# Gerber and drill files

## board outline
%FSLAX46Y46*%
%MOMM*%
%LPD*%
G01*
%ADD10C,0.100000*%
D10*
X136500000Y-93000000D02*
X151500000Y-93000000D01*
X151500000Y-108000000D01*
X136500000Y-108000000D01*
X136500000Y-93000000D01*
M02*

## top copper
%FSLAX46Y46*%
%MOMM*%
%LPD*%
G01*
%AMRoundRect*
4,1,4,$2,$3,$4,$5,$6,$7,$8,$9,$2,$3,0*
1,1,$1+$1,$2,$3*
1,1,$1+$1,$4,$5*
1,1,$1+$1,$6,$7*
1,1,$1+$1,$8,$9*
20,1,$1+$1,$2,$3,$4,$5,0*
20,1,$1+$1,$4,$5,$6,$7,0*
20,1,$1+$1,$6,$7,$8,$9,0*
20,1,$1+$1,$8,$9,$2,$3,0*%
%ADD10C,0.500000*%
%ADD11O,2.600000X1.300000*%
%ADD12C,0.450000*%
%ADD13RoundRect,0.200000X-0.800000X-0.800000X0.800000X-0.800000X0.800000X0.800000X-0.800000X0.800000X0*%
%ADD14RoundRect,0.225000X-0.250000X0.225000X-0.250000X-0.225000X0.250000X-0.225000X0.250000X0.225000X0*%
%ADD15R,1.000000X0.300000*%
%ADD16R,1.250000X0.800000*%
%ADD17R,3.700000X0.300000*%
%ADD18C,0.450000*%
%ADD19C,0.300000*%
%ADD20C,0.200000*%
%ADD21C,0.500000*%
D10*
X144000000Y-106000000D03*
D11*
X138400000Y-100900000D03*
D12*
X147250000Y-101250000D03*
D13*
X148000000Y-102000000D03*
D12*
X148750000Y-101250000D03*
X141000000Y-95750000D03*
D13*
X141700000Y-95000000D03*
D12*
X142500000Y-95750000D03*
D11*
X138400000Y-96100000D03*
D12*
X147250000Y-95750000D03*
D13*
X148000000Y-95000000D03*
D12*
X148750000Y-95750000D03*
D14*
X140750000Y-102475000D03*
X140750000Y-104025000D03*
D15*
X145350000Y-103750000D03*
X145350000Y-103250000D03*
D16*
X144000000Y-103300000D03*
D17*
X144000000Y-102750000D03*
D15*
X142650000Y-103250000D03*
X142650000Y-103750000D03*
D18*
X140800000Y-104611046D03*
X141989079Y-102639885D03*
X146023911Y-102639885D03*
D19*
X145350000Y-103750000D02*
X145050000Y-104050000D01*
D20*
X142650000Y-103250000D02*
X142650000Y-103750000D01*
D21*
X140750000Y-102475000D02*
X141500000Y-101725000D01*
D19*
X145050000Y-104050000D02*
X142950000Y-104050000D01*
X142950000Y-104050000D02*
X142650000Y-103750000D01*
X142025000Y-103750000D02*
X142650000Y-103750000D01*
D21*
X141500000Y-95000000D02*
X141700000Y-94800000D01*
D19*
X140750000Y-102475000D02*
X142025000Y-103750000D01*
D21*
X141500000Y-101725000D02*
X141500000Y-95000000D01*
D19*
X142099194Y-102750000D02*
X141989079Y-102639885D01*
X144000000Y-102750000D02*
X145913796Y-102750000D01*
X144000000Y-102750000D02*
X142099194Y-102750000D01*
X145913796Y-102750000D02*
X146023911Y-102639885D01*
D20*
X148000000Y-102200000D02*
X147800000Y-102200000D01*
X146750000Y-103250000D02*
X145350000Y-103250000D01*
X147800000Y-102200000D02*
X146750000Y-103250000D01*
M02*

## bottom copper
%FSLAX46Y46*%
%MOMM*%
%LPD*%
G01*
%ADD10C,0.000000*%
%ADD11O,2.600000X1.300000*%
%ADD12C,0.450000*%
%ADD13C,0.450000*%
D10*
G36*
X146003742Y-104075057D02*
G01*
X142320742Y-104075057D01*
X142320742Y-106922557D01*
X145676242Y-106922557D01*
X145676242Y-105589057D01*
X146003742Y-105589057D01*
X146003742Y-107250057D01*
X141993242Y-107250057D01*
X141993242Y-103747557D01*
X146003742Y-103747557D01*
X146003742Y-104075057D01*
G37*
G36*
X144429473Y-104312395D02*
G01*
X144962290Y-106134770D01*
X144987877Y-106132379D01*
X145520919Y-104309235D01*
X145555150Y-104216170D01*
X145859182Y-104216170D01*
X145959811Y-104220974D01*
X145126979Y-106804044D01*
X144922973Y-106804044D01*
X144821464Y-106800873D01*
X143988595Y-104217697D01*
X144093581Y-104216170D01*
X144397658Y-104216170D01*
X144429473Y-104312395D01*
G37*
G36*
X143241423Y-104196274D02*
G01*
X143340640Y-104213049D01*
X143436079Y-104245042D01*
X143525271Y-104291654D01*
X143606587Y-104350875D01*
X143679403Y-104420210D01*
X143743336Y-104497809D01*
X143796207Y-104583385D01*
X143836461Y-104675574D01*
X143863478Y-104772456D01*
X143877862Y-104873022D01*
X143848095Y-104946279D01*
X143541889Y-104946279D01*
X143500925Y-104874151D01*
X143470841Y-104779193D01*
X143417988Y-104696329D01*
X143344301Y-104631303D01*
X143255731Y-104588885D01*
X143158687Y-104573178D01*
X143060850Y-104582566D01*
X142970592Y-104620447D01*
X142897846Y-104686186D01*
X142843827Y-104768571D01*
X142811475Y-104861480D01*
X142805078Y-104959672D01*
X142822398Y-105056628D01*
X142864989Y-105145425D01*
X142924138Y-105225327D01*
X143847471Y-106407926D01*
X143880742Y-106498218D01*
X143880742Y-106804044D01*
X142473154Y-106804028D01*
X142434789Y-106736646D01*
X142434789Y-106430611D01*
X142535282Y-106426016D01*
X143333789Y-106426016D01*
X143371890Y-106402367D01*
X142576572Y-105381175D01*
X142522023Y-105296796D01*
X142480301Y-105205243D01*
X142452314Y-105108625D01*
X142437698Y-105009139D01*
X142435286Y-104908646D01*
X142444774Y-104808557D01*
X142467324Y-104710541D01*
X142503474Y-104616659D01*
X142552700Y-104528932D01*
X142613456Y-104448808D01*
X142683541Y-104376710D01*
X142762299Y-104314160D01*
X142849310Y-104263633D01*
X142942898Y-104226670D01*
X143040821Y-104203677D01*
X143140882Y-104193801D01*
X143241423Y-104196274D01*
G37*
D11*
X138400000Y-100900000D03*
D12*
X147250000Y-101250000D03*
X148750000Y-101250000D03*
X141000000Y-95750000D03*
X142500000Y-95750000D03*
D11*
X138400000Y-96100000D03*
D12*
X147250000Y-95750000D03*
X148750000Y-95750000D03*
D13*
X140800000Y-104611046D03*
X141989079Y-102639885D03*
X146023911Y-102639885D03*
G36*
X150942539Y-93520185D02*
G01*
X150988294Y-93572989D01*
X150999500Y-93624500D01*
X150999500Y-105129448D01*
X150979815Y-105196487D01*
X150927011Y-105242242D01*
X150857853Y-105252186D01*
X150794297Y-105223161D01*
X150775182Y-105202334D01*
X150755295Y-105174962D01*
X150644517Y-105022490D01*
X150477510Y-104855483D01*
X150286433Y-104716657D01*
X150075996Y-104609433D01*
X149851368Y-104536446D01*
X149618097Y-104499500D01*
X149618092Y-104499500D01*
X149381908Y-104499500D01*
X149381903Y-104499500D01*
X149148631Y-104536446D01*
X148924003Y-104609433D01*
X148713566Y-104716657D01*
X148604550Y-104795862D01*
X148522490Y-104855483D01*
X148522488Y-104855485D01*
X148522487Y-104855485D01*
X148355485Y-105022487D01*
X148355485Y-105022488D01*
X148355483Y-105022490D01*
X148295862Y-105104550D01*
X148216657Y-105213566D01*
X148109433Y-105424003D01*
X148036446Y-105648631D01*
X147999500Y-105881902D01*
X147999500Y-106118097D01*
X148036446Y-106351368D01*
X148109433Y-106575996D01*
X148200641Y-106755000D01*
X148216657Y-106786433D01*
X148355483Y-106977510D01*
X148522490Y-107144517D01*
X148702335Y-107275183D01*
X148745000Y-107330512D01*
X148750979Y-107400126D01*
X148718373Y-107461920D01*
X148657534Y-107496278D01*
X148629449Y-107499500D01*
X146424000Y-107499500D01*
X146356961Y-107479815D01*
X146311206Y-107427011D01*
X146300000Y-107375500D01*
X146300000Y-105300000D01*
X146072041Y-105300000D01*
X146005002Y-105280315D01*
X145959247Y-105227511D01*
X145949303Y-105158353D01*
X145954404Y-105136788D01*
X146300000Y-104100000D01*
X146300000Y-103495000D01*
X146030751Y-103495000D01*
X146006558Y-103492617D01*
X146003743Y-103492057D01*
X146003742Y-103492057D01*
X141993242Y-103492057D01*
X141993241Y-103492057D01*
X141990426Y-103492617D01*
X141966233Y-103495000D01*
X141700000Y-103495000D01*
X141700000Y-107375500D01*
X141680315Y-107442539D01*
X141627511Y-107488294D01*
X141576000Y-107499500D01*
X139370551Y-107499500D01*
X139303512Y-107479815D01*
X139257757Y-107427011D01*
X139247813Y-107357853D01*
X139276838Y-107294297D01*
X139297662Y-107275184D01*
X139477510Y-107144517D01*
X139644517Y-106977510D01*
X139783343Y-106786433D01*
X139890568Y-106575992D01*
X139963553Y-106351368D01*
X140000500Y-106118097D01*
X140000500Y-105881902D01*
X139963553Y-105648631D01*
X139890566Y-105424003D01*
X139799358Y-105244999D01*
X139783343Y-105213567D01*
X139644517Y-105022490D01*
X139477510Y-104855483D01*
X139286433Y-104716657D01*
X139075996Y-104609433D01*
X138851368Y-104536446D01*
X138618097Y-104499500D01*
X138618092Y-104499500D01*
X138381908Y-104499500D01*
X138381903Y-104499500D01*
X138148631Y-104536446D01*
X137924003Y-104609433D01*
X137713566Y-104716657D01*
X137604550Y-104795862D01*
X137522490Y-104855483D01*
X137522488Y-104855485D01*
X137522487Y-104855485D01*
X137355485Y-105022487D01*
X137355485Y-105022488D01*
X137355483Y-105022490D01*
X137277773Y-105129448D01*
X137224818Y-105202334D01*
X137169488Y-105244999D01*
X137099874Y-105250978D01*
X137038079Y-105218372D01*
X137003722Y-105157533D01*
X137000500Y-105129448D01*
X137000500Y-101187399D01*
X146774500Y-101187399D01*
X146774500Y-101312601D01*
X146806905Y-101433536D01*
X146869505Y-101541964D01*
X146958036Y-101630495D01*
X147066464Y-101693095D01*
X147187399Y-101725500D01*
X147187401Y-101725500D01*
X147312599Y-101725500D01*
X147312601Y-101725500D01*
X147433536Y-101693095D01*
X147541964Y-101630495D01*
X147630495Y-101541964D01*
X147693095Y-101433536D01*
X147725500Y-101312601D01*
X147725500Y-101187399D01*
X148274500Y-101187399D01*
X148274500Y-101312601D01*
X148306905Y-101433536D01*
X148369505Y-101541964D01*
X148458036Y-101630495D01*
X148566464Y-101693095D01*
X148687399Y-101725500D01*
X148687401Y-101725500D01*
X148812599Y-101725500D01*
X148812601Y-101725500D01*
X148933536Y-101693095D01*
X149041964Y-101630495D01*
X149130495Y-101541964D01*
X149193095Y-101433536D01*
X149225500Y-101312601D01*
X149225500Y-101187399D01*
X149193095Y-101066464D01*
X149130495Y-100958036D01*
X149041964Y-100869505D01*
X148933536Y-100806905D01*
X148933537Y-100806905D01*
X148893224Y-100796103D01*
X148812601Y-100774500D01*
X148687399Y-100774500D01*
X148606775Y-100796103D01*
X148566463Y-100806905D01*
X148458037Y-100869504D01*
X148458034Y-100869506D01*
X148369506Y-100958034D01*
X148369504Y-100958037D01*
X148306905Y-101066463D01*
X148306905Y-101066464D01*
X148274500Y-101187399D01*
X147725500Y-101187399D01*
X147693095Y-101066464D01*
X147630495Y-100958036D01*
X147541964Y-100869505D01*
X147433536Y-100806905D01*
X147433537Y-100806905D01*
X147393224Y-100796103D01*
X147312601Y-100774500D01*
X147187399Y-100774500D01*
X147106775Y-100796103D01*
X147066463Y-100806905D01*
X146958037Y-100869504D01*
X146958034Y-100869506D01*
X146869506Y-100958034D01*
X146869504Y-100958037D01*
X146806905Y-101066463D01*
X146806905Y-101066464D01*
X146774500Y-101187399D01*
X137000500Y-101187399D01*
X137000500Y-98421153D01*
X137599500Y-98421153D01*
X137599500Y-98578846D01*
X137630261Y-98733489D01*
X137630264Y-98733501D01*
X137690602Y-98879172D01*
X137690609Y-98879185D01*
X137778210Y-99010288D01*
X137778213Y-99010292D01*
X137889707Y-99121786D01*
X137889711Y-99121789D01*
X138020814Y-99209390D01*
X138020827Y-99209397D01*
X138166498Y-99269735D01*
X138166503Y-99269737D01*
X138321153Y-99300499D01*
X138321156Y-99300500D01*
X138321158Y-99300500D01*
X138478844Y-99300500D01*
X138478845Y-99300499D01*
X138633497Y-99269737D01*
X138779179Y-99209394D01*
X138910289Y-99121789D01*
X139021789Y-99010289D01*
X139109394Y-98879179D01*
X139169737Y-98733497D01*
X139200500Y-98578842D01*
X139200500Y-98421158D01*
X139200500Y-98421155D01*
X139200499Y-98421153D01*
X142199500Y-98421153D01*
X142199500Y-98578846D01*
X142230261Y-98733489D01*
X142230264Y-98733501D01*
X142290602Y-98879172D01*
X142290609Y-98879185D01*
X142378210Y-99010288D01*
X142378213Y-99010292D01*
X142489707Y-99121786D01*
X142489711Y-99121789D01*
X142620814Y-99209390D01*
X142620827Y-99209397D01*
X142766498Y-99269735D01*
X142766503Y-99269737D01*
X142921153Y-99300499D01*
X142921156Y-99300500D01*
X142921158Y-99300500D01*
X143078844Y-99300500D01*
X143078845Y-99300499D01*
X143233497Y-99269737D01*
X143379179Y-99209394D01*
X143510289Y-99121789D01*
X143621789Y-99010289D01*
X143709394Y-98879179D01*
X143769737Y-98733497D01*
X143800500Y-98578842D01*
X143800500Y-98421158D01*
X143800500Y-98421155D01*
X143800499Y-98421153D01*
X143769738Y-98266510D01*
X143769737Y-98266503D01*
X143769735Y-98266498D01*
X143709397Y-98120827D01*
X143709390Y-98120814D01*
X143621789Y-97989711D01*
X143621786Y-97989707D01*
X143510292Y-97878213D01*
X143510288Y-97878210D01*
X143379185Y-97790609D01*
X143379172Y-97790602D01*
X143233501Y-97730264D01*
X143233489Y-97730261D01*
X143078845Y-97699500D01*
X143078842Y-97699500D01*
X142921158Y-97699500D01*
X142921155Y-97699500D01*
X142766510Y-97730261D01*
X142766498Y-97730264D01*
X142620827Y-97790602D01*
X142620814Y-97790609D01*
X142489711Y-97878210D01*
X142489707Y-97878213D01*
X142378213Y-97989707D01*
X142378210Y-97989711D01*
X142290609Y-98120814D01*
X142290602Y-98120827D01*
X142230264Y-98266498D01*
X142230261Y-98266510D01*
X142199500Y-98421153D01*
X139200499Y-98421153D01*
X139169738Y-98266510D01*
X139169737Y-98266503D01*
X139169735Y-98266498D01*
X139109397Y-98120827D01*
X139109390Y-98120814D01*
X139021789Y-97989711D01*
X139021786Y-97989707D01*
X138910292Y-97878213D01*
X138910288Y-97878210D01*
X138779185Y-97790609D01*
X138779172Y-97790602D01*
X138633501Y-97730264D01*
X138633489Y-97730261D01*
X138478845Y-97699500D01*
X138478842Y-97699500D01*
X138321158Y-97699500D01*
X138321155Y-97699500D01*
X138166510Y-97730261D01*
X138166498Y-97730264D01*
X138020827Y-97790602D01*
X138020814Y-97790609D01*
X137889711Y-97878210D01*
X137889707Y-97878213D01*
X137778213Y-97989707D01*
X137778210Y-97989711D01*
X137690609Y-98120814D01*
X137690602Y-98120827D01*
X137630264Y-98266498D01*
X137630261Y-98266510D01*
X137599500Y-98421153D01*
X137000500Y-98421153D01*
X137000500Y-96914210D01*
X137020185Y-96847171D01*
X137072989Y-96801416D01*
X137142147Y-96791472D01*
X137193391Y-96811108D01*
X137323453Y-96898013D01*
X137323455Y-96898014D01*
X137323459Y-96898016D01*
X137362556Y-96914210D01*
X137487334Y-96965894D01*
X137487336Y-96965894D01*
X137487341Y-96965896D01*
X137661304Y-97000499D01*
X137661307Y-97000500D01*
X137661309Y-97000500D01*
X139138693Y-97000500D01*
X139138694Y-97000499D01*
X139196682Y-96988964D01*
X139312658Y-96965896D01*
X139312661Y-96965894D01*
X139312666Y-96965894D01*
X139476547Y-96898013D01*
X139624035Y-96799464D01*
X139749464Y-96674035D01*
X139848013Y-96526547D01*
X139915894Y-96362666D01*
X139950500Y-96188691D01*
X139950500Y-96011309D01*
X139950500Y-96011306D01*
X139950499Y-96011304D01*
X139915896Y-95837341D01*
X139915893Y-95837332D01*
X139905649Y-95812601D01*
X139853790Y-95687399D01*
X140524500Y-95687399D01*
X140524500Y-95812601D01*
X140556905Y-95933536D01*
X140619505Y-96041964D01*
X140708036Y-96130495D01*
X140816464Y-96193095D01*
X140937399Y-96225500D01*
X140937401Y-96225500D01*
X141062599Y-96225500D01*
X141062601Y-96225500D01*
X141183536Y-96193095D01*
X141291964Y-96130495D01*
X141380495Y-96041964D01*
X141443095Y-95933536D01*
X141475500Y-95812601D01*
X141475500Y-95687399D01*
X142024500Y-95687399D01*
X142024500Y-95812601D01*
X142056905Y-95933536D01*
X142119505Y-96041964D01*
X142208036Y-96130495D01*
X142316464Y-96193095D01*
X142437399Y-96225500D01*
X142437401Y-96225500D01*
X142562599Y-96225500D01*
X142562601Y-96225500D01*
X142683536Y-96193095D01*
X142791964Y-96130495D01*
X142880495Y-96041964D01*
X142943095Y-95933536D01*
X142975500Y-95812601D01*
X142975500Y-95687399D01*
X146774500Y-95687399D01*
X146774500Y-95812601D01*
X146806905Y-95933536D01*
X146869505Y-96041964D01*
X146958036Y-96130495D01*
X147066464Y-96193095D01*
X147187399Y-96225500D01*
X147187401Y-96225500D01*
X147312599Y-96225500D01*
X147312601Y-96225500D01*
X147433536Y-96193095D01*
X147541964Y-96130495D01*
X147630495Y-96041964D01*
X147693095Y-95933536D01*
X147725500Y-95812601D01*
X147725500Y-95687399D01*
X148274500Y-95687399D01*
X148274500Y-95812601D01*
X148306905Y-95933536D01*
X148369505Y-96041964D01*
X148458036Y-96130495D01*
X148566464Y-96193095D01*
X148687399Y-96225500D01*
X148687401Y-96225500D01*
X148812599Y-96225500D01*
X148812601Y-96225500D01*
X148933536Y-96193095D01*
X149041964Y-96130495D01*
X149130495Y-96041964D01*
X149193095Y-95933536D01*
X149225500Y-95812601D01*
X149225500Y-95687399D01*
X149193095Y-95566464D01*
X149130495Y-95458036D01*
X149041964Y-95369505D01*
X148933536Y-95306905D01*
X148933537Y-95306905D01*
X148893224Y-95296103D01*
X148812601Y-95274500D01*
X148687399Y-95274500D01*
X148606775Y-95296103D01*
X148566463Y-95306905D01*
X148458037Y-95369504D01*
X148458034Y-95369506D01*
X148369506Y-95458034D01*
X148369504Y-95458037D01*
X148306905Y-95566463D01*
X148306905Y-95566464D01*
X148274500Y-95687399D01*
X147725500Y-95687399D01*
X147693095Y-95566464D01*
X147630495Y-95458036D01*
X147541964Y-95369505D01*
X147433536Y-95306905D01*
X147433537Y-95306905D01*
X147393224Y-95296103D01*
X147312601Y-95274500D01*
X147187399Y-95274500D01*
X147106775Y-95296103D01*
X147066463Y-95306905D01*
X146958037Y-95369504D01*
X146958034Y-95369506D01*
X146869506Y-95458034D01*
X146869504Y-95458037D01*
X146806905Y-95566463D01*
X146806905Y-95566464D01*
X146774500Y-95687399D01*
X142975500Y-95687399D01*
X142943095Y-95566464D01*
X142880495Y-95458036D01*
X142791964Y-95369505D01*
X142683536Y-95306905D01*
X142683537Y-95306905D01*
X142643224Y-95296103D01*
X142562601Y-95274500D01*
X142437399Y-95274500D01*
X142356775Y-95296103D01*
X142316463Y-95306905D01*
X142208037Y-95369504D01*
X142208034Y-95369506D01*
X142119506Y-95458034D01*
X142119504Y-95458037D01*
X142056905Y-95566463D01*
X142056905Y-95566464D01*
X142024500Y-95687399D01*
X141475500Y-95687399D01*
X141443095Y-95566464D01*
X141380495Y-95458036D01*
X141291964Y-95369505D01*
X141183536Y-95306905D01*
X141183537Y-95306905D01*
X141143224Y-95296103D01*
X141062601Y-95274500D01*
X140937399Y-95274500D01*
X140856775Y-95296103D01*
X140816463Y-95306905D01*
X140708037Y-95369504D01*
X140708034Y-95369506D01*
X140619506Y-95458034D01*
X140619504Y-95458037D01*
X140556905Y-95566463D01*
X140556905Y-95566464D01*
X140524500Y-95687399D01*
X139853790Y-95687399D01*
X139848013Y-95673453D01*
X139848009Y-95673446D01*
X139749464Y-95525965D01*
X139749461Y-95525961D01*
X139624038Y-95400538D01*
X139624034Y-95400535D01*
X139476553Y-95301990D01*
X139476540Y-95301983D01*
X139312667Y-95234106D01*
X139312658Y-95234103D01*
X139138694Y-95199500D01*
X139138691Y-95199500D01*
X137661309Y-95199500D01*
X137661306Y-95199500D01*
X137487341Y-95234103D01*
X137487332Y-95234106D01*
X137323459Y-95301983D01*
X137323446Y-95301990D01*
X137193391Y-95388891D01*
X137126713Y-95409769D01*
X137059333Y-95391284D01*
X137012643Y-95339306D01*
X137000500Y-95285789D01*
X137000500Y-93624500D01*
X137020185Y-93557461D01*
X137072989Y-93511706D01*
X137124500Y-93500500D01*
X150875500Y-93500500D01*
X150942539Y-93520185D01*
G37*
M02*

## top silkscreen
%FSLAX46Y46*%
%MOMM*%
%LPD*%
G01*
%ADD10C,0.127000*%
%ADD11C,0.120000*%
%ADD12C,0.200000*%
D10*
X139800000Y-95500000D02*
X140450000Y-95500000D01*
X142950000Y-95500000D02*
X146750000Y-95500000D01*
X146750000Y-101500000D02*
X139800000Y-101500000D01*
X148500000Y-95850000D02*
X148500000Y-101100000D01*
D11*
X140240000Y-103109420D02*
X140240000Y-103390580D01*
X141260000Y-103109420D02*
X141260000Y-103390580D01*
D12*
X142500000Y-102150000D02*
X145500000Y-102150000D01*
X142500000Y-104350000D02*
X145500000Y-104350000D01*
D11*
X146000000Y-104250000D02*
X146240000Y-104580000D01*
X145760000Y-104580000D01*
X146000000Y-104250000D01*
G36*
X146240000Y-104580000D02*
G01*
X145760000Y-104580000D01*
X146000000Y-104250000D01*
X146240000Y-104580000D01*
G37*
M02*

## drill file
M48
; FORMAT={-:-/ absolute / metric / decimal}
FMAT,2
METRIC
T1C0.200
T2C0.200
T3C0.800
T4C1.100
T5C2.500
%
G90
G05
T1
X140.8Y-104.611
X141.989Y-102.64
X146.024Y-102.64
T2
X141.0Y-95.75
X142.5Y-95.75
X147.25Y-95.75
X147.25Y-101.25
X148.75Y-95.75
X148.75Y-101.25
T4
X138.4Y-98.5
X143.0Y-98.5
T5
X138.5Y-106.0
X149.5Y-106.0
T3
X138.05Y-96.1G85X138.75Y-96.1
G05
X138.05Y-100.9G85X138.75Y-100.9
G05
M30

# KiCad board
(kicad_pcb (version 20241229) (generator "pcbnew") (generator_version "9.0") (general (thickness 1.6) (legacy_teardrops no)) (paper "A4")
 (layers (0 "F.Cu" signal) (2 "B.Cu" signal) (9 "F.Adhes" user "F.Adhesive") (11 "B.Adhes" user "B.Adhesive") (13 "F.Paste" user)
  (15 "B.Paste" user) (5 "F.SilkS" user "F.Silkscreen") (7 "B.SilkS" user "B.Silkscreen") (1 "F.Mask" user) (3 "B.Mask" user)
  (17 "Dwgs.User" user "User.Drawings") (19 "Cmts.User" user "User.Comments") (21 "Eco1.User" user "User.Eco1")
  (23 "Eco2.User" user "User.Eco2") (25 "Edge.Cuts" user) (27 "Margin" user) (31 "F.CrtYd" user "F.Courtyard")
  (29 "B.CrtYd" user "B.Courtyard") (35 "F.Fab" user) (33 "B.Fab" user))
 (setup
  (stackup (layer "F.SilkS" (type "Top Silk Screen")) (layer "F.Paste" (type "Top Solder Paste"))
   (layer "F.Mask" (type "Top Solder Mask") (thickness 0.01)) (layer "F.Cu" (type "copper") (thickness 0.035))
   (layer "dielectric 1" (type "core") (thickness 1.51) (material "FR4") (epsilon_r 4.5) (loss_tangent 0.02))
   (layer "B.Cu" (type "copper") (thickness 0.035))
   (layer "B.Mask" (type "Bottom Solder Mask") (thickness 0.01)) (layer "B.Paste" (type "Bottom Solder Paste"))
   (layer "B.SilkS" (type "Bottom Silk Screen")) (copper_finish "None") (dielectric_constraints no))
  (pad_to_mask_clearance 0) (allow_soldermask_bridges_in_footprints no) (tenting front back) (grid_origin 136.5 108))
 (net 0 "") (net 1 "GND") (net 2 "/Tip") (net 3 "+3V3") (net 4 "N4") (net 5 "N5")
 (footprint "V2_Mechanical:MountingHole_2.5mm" (layer "F.Cu") (at 138.5 106)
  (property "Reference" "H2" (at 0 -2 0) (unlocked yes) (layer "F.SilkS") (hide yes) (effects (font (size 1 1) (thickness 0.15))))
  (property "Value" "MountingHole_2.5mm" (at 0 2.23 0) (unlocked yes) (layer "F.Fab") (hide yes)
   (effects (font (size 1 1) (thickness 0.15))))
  (pad "" np_thru_hole circle (at 0 0) (size 2.5 2.5) (drill 2.5) (layers "*.Mask")))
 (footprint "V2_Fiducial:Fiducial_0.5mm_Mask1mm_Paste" (layer "F.Cu") (at 144 106)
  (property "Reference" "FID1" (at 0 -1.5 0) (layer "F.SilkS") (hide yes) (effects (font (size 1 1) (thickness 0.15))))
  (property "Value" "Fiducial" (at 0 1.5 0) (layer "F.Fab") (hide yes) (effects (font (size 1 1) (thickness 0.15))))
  (pad "" smd circle (at 0 0) (size 0.5 0.5) (layers "F.Cu" "F.Mask" "F.Paste") (solder_mask_margin 0.25) (clearance 0.25)))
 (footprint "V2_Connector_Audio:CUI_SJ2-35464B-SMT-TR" (layer "F.Cu") (at 142.5 98.5)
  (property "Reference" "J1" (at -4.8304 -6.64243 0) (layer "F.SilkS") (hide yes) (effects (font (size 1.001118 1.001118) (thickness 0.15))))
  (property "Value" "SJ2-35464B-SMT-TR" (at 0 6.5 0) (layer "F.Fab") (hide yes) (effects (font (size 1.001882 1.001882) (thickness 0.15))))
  (fp_line (start -2.7 -3) (end -2.05 -3) (stroke (width 0.127) (type solid)) (layer "F.SilkS"))
  (fp_line (start 0.45 -3) (end 4.25 -3) (stroke (width 0.127) (type solid)) (layer "F.SilkS"))
  (fp_line (start 4.25 3) (end -2.7 3) (stroke (width 0.127) (type solid)) (layer "F.SilkS"))
  (fp_line (start 6 -2.65) (end 6 2.6) (stroke (width 0.127) (type solid)) (layer "F.SilkS"))
  (pad "" np_thru_hole circle (at -4.1 0) (size 1.1 1.1) (drill 1.1) (layers "*.Cu" "*.Mask"))
  (pad "" smd roundrect (at -0.8 -3.7) (size 2 1.6) (layers "F.Mask") (roundrect_rratio 0.1) (solder_mask_margin 0.102))
  (pad "" smd roundrect (at -0.75 -3.825) (size 2.5 1.85) (layers "F.Paste") (roundrect_rratio 0.25) (solder_mask_margin 0.102))
  (pad "" np_thru_hole circle (at 0.5 0) (size 1.1 1.1) (drill 1.1) (layers "*.Cu" "*.Mask"))
  (pad "" smd roundrect (at 5.5 -3.825) (size 2.5 1.85) (layers "F.Paste") (roundrect_rratio 0.25) (solder_mask_margin 0.102))
  (pad "" smd roundrect (at 5.5 -3.7) (size 2 1.6) (layers "F.Mask") (roundrect_rratio 0.1) (solder_mask_margin 0.102))
  (pad "" smd roundrect (at 5.5 3.7) (size 2 1.6) (layers "F.Mask") (roundrect_rratio 0.1) (solder_mask_margin 0.102))
  (pad "" smd roundrect (at 5.5 3.825) (size 2.5 1.85) (layers "F.Paste") (roundrect_rratio 0.25) (solder_mask_margin 0.102))
  (pad "1" thru_hole oval (at -4.1 2.4) (size 2.6 1.3) (drill oval 1.5 0.8) (layers "*.Cu" "F.Mask" "F.Paste") (remove_unused_layers yes)
   (keep_end_layers yes) (zone_layer_connections) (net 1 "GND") (solder_mask_margin 0.102))
  (pad "2" thru_hole circle (at 4.75 2.75) (size 0.45 0.45) (drill 0.2) (layers "*.Cu") (remove_unused_layers yes) (keep_end_layers yes)
   (zone_layer_connections) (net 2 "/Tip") (solder_mask_margin 0.102))
  (pad "2" smd roundrect (at 5.5 3.5) (size 2 2) (layers "F.Cu") (roundrect_rratio 0.1) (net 2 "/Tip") (solder_mask_margin 0.102))
  (pad "2" thru_hole circle (at 6.25 2.75) (size 0.45 0.45) (drill 0.2) (layers "*.Cu") (remove_unused_layers yes) (keep_end_layers yes)
   (zone_layer_connections) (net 2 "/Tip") (solder_mask_margin 0.102))
  (pad "3" thru_hole circle (at -1.5 -2.75) (size 0.45 0.45) (drill 0.2) (layers "*.Cu") (remove_unused_layers yes) (keep_end_layers yes)
   (zone_layer_connections) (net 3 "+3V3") (solder_mask_margin 0.102))
  (pad "3" smd roundrect (at -0.8 -3.5) (size 2 2) (layers "F.Cu") (roundrect_rratio 0.1) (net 3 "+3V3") (solder_mask_margin 0.102))
  (pad "3" thru_hole circle (at 0 -2.75) (size 0.45 0.45) (drill 0.2) (layers "*.Cu") (remove_unused_layers yes) (keep_end_layers yes)
   (zone_layer_connections) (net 3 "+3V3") (solder_mask_margin 0.102))
  (pad "4" thru_hole oval (at -4.1 -2.4) (size 2.6 1.3) (drill oval 1.5 0.8) (layers "*.Cu" "F.Mask" "F.Paste") (remove_unused_layers yes)
   (keep_end_layers yes) (zone_layer_connections) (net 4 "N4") (solder_mask_margin 0.102))
  (pad "10" thru_hole circle (at 4.75 -2.75) (size 0.45 0.45) (drill 0.2) (layers "*.Cu") (remove_unused_layers yes) (keep_end_layers yes)
   (zone_layer_connections) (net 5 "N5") (solder_mask_margin 0.102))
  (pad "10" smd roundrect (at 5.5 -3.5) (size 2 2) (layers "F.Cu") (roundrect_rratio 0.1) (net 5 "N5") (solder_mask_margin 0.102))
  (pad "10" thru_hole circle (at 6.25 -2.75) (size 0.45 0.45) (drill 0.2) (layers "*.Cu") (remove_unused_layers yes) (keep_end_layers yes)
   (zone_layer_connections) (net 5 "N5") (solder_mask_margin 0.102)))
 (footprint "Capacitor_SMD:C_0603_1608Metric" (layer "F.Cu") (at 140.75 103.25 -90)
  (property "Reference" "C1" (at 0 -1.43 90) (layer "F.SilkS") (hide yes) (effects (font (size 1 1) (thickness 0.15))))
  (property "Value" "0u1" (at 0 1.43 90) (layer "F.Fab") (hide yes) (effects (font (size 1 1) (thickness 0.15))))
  (fp_line (start -0.14058 0.51) (end 0.14058 0.51) (stroke (width 0.12) (type solid)) (layer "F.SilkS"))
  (fp_line (start -0.14058 -0.51) (end 0.14058 -0.51) (stroke (width 0.12) (type solid)) (layer "F.SilkS"))
  (pad "1" smd roundrect (at -0.775 0 270) (size 0.9 0.95) (layers "F.Cu" "F.Mask" "F.Paste") (roundrect_rratio 0.25) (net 3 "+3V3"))
  (pad "2" smd roundrect (at 0.775 0 270) (size 0.9 0.95) (layers "F.Cu" "F.Mask" "F.Paste") (roundrect_rratio 0.25) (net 1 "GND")))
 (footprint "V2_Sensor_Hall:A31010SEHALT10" (layer "F.Cu") (at 144 103.25 90)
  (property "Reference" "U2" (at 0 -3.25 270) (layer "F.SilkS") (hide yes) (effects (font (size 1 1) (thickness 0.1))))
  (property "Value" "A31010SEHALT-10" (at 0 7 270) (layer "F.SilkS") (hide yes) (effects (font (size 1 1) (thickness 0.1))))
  (fp_line (start 1.1 -1.5) (end 1.1 1.5) (stroke (width 0.2) (type solid)) (layer "F.SilkS"))
  (fp_line (start -1.1 -1.5) (end -1.1 1.5) (stroke (width 0.2) (type solid)) (layer "F.SilkS"))
  (fp_poly (pts (xy -1 2) (xy -1.33 2.24) (xy -1.33 1.76) (xy -1 2)) (stroke (width 0.12) (type solid)) (fill yes) (layer "F.SilkS"))
  (pad "" smd rect (at -0.22144 0.351384 90) (size 0.44288 0.502768) (layers "F.Paste"))
  (pad "" smd rect (at -0.221438 -0.357879 90) (size 0.442876 0.515758) (layers "F.Paste"))
  (pad "" smd rect (at 0.430523 -0.357878 90) (size 0.437668 0.515756) (layers "F.Paste"))
  (pad "" smd rect (at 0.430523 0.351385 90) (size 0.437668 0.50277) (layers "F.Paste"))
  (pad "" smd rect (at 0.5 -1.35 90) (size 0.3 1) (layers "F.Paste"))
  (pad "" smd rect (at 0.5 1.35 90) (size 0.3 1) (layers "F.Paste"))
  (pad "1" smd rect (at -0.5 1.35 90) (size 0.3 1) (layers "F.Cu" "F.Mask" "F.Paste") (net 3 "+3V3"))
  (pad "2" smd rect (at 0 1.35 90) (size 0.3 1) (layers "F.Cu" "F.Mask" "F.Paste") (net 2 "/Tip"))
  (pad "3" smd rect (at -0.05 0 90) (size 0.8 1.25) (layers "F.Cu" "F.Mask") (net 1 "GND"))
  (pad "3" smd rect (at 0.5 0 90) (size 0.3 3.7) (layers "F.Cu" "F.Mask") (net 1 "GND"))
  (pad "5" smd rect (at 0 -1.35 90) (size 0.3 1) (layers "F.Cu" "F.Mask" "F.Paste") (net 3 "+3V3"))
  (pad "6" smd rect (at -0.5 -1.35 90) (size 0.3 1) (layers "F.Cu" "F.Mask" "F.Paste") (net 3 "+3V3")))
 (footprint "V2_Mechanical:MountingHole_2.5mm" (layer "F.Cu") (at 149.5 106)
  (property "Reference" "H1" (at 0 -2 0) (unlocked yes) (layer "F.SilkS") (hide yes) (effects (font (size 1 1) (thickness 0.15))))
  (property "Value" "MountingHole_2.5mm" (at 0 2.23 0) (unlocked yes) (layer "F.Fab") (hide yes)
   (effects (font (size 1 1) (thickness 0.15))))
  (pad "" np_thru_hole circle (at 0 0) (size 2.5 2.5) (drill 2.5) (layers "*.Mask")))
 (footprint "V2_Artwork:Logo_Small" (layer "B.Cu") (at 144 105.5 180)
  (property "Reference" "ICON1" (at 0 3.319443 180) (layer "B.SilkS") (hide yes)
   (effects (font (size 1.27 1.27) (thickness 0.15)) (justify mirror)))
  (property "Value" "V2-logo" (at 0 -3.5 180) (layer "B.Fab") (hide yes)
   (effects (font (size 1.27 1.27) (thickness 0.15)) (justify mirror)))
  (fp_poly
   (pts (xy 2.006758 -1.750057) (xy -2.003742 -1.750057) (xy -2.003742 -0.089057) (xy -1.676242 -0.089057) (xy -1.676242 -1.422557)
    (xy 1.679258 -1.422557) (xy 1.679258 1.424943) (xy -2.003742 1.424943) (xy -2.003742 1.752443) (xy 2.006758 1.752443))
   (stroke (width 0) (type solid)) (fill yes) (layer "B.Cu"))
  (fp_poly
   (pts (xy -1.520919 1.190765) (xy -0.987877 -0.632379) (xy -0.96229 -0.63477) (xy -0.429473 1.187605) (xy -0.397658 1.28383)
    (xy -0.093581 1.28383) (xy 0.011405 1.282303) (xy -0.821464 -1.300873) (xy -0.922973 -1.304044) (xy -1.126979 -1.304044)
    (xy -1.959811 1.279026) (xy -1.859182 1.28383) (xy -1.55515 1.28383))
   (stroke (width 0) (type solid)) (fill yes) (layer "B.Cu"))
  (fp_poly
   (pts (xy 0.959179 1.296323) (xy 1.057102 1.27333) (xy 1.15069 1.236367) (xy 1.237701 1.18584) (xy 1.316459 1.12329)
    (xy 1.386544 1.051192) (xy 1.4473 0.971068) (xy 1.496526 0.883341) (xy 1.532676 0.789459) (xy 1.555226 0.691443) (xy 1.564714 0.591354)
    (xy 1.562302 0.490861) (xy 1.547686 0.391375) (xy 1.519699 0.294757) (xy 1.477977 0.203204) (xy 1.423428 0.118825)
    (xy 0.62811 -0.902367) (xy 0.666211 -0.926016) (xy 1.464718 -0.926016) (xy 1.565211 -0.930611) (xy 1.565211 -1.236646)
    (xy 1.526846 -1.304028) (xy 0.119258 -1.304044) (xy 0.119258 -0.998218) (xy 0.152529 -0.907926) (xy 1.075862 0.274673)
    (xy 1.135011 0.354575) (xy 1.177602 0.443372) (xy 1.194922 0.540328) (xy 1.188525 0.63852) (xy 1.156173 0.731429) (xy 1.102154 0.813814)
    (xy 1.029408 0.879553) (xy 0.93915 0.917434) (xy 0.841313 0.926822) (xy 0.744269 0.911115) (xy 0.655699 0.868697) (xy 0.582012 0.803671)
    (xy 0.529159 0.720807) (xy 0.499075 0.625849) (xy 0.458111 0.553721) (xy 0.151905 0.553721) (xy 0.122138 0.626978)
    (xy 0.136522 0.727544) (xy 0.163539 0.824426) (xy 0.203793 0.916615) (xy 0.256664 1.002191) (xy 0.320597 1.07979) (xy 0.393413 1.149125)
    (xy 0.474729 1.208346) (xy 0.563921 1.254958) (xy 0.65936 1.286951) (xy 0.758577 1.303726) (xy 0.859118 1.306199))
   (stroke (width 0) (type solid)) (fill yes) (layer "B.Cu"))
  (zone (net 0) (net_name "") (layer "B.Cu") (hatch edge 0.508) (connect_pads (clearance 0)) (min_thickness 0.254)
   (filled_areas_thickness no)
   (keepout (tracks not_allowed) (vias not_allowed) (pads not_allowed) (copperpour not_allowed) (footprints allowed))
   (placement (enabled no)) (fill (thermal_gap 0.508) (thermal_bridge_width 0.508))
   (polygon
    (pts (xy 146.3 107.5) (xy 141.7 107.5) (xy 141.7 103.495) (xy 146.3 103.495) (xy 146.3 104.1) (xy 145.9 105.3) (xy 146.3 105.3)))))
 (gr_rect (start 136.5 93) (end 151.5 108) (stroke (width 0.1) (type default)) (fill no) (layer "Edge.Cuts"))
 (segment (start 145.35 103.75) (end 145.05 104.05) (width 0.3) (layer "F.Cu") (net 3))
 (segment (start 142.65 103.25) (end 142.65 103.75) (width 0.2) (layer "F.Cu") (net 3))
 (segment (start 140.75 102.475) (end 141.5 101.725) (width 0.5) (layer "F.Cu") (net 3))
 (segment (start 145.05 104.05) (end 142.95 104.05) (width 0.3) (layer "F.Cu") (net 3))
 (segment (start 142.95 104.05) (end 142.65 103.75) (width 0.3) (layer "F.Cu") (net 3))
 (segment (start 142.025 103.75) (end 142.65 103.75) (width 0.3) (layer "F.Cu") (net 3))
 (segment (start 141.5 95) (end 141.7 94.8) (width 0.5) (layer "F.Cu") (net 3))
 (segment (start 140.75 102.475) (end 142.025 103.75) (width 0.3) (layer "F.Cu") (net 3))
 (segment (start 141.5 101.725) (end 141.5 95) (width 0.5) (layer "F.Cu") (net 3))
 (segment (start 142.099194 102.75) (end 141.989079 102.639885) (width 0.3) (layer "F.Cu") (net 1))
 (segment (start 144 102.75) (end 145.913796 102.75) (width 0.3) (layer "F.Cu") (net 1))
 (segment (start 144 102.75) (end 142.099194 102.75) (width 0.3) (layer "F.Cu") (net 1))
 (segment (start 145.913796 102.75) (end 146.023911 102.639885) (width 0.3) (layer "F.Cu") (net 1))
 (via (at 140.8 104.611046) (size 0.45) (drill 0.2) (layers "F.Cu" "B.Cu") (free yes) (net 1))
 (via (at 141.989079 102.639885) (size 0.45) (drill 0.2) (layers "F.Cu" "B.Cu") (free yes) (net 1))
 (via (at 146.023911 102.639885) (size 0.45) (drill 0.2) (layers "F.Cu" "B.Cu") (free yes) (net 1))
 (segment (start 148 102.2) (end 147.8 102.2) (width 0.2) (layer "F.Cu") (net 2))
 (segment (start 146.75 103.25) (end 145.35 103.25) (width 0.2) (layer "F.Cu") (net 2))
 (segment (start 147.8 102.2) (end 146.75 103.25) (width 0.2) (layer "F.Cu") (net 2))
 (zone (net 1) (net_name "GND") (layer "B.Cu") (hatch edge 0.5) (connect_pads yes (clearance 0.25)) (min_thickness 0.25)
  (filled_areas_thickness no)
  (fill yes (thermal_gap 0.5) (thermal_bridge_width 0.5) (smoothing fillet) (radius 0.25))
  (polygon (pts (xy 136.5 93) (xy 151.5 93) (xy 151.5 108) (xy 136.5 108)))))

